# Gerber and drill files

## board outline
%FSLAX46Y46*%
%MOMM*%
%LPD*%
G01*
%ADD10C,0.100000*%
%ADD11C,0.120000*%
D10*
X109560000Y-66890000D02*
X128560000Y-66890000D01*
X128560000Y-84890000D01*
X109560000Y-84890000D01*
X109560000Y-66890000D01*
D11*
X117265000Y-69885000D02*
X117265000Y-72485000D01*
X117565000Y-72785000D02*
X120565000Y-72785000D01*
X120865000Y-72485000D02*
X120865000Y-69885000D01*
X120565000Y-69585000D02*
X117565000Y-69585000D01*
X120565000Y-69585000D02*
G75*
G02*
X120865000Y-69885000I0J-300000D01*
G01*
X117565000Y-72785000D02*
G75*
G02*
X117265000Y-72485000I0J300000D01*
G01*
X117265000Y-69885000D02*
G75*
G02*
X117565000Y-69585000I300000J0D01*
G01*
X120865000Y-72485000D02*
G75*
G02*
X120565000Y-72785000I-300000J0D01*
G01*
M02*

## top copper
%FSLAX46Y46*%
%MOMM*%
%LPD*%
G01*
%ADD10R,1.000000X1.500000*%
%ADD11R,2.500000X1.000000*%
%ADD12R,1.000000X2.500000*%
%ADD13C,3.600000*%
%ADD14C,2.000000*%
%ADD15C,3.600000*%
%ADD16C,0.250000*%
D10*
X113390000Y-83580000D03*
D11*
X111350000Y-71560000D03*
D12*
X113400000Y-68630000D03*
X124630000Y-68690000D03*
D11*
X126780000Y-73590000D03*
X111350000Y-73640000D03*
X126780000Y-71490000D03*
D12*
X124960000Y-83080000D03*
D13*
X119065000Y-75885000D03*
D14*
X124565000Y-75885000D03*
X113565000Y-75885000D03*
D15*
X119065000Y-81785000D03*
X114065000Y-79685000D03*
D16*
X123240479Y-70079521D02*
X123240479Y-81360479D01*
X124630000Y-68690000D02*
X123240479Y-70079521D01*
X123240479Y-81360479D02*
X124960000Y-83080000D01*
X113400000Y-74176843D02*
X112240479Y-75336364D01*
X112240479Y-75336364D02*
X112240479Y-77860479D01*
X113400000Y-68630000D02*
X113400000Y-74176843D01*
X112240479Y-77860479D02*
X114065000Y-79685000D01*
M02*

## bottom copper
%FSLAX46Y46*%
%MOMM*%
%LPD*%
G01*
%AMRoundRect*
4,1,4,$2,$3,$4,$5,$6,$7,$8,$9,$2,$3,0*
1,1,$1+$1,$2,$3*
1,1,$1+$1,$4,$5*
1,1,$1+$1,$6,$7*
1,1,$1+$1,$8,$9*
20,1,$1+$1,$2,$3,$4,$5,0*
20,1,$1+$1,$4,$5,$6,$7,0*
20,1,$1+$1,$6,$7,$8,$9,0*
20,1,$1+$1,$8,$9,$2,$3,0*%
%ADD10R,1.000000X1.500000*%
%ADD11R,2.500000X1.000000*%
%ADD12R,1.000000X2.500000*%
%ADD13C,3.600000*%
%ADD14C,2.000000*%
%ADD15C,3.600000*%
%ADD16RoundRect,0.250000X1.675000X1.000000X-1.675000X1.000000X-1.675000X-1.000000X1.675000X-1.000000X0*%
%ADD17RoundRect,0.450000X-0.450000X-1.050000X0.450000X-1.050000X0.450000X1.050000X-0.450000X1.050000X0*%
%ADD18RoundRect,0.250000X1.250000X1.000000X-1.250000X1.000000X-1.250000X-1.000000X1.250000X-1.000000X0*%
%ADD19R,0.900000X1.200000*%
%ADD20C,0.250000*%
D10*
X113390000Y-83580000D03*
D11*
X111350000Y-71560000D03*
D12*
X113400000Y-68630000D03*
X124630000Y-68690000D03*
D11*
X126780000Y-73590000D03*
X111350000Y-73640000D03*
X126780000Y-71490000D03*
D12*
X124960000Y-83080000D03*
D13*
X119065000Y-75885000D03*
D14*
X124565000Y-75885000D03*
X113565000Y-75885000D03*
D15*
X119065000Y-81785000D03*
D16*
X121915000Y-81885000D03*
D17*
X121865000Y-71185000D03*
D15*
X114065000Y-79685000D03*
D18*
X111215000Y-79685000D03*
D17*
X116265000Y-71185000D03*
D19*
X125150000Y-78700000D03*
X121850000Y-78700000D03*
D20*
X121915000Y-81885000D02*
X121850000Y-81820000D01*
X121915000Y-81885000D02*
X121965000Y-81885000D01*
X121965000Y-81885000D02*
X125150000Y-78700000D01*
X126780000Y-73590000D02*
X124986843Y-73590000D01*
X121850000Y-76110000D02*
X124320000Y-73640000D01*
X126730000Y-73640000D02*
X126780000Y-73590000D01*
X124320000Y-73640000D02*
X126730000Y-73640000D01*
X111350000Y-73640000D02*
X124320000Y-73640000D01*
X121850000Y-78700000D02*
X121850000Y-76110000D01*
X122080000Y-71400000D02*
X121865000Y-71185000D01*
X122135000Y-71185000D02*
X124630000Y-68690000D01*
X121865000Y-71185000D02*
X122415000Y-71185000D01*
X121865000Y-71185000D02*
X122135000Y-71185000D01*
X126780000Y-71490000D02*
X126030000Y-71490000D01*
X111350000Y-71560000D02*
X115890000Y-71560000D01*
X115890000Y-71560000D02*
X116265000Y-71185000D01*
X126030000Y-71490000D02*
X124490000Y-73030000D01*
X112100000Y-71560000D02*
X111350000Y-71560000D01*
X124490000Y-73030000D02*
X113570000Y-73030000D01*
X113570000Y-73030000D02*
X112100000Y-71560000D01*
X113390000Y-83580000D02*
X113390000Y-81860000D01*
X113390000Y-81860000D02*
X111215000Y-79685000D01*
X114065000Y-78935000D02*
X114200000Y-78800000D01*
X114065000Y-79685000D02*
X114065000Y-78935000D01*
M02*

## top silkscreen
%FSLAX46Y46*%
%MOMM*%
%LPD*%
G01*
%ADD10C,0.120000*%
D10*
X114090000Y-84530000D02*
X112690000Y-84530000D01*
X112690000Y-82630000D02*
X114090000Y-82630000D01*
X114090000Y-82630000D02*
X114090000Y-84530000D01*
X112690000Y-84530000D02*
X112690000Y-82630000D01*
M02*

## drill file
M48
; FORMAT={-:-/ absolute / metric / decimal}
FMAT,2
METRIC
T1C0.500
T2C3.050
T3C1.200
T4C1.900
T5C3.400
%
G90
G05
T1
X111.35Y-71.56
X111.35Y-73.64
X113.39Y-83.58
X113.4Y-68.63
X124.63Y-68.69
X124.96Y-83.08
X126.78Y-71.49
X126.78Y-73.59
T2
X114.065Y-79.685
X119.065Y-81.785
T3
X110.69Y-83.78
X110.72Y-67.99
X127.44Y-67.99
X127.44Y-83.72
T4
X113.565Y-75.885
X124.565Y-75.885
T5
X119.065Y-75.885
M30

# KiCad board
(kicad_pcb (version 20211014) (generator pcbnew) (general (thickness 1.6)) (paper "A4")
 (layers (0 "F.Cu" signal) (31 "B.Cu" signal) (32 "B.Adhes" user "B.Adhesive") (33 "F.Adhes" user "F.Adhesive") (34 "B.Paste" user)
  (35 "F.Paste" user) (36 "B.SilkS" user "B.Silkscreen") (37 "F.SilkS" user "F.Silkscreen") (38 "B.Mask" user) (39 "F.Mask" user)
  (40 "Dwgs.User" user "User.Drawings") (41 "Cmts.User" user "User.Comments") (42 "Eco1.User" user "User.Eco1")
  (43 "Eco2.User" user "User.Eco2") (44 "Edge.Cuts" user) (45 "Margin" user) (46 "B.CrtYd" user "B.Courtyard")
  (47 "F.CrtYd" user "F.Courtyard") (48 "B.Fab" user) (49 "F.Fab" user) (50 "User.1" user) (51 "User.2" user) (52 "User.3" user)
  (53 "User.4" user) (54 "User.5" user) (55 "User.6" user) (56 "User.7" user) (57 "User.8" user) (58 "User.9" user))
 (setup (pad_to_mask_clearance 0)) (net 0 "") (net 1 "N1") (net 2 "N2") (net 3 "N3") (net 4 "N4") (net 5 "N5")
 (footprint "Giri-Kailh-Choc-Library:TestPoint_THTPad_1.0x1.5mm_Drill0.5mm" (layer "F.Cu") (at 113.39 83.58 -90)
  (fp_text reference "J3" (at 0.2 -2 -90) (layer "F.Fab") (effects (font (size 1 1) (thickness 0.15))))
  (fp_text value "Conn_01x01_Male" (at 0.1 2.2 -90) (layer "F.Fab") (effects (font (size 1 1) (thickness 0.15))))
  (fp_line (start 0.95 -0.7) (end 0.95 0.7) (layer "F.SilkS") (width 0.12))
  (fp_line (start -0.95 0.7) (end -0.95 -0.7) (layer "F.SilkS") (width 0.12))
  (fp_line (start -0.95 -0.7) (end 0.95 -0.7) (layer "F.SilkS") (width 0.12))
  (fp_line (start 0.95 0.7) (end -0.95 0.7) (layer "F.SilkS") (width 0.12))
  (pad "1" thru_hole rect (at 0 0 270) (size 1.5 1) (drill 0.5) (layers *.Cu *.Mask) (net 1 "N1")))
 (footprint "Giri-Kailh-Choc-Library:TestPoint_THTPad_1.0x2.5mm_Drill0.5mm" (layer "F.Cu") (at 111.35 71.56)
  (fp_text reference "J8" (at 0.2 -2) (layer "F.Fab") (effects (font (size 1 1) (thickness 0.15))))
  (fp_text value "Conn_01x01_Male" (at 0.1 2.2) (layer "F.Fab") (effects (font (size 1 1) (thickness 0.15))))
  (pad "1" thru_hole rect (at 0 0) (size 2.5 1) (drill 0.5) (layers *.Cu *.Mask) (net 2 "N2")))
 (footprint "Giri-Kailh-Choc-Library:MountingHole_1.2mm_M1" (layer "F.Cu") (at 110.69 83.78)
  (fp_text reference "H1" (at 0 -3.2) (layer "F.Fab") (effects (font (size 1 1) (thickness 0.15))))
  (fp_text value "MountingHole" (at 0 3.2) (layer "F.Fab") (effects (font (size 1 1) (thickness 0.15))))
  (pad "" np_thru_hole circle (at 0 0) (size 1.2 1.2) (drill 1.2) (layers F&B.Cu *.Mask)))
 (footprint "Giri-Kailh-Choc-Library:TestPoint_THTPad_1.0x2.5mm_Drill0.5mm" (layer "F.Cu") (at 113.4 68.63 90)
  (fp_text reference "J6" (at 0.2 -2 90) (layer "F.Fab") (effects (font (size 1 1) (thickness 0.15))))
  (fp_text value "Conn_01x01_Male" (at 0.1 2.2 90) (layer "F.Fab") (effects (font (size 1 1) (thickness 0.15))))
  (pad "1" thru_hole rect (at 0 0 90) (size 2.5 1) (drill 0.5) (layers *.Cu *.Mask) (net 1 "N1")))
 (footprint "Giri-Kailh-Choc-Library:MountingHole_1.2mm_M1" (layer "F.Cu") (at 127.44 83.72)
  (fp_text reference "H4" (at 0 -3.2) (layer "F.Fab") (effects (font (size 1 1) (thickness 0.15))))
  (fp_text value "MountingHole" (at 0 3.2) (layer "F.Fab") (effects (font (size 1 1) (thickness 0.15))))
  (pad "" np_thru_hole circle (at 0 0) (size 1.2 1.2) (drill 1.2) (layers F&B.Cu *.Mask)))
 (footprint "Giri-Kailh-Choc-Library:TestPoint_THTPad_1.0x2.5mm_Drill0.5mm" (layer "F.Cu") (at 124.63 68.69 90)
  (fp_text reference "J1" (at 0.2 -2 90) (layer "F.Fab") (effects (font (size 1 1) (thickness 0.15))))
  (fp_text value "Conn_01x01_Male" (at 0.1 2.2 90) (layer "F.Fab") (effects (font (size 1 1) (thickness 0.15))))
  (pad "1" thru_hole rect (at 0 0 90) (size 2.5 1) (drill 0.5) (layers *.Cu *.Mask) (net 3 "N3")))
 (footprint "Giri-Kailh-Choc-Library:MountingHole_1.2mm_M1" (layer "F.Cu") (at 127.44 67.99)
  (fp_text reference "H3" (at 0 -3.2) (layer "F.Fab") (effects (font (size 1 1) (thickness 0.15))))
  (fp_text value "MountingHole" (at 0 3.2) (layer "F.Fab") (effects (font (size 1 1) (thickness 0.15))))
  (pad "" np_thru_hole circle (at 0 0) (size 1.2 1.2) (drill 1.2) (layers F&B.Cu *.Mask)))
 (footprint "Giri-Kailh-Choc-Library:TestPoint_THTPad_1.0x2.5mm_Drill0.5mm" (layer "F.Cu") (at 126.78 73.59)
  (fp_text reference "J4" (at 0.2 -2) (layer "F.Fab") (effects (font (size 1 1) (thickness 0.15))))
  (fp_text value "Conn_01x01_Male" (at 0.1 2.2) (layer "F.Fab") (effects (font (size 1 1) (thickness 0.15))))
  (pad "1" thru_hole rect (at 0 0) (size 2.5 1) (drill 0.5) (layers *.Cu *.Mask) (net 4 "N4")))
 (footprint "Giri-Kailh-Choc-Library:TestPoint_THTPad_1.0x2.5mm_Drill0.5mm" (layer "F.Cu") (at 111.35 73.64)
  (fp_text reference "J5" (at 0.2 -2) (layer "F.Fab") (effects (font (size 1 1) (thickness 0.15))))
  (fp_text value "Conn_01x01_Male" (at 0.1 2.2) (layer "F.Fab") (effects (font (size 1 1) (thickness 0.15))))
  (pad "1" thru_hole rect (at 0 0) (size 2.5 1) (drill 0.5) (layers *.Cu *.Mask) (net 4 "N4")))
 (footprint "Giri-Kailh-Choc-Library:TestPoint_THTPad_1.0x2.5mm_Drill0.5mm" (layer "F.Cu") (at 126.78 71.49)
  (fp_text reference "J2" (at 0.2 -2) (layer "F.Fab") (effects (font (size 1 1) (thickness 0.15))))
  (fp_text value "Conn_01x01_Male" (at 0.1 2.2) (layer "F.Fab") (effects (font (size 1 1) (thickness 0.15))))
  (pad "1" thru_hole rect (at 0 0) (size 2.5 1) (drill 0.5) (layers *.Cu *.Mask) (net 2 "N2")))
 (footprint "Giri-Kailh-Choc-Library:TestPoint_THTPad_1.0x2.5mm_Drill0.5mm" (layer "F.Cu") (at 124.96 83.08 90)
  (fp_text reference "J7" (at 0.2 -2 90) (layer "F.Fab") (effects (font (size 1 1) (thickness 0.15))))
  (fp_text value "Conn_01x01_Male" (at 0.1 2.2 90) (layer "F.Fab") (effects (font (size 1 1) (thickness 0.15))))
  (pad "1" thru_hole rect (at 0 0 90) (size 2.5 1) (drill 0.5) (layers *.Cu *.Mask) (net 3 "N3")))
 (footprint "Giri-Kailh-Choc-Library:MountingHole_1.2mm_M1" (layer "F.Cu") (at 110.72 67.99)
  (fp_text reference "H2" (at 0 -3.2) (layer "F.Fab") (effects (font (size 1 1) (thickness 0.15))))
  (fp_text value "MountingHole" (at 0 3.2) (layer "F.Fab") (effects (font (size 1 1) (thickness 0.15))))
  (pad "" np_thru_hole circle (at 0 0) (size 1.2 1.2) (drill 1.2) (layers F&B.Cu *.Mask)))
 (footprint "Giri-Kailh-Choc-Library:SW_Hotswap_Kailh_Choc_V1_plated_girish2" (layer "F.Cu") (at 119.065 75.885)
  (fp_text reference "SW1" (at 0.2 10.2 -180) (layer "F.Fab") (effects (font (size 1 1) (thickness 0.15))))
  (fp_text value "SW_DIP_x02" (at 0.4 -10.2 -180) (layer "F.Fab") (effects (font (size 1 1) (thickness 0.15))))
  (fp_line (start -1.8 -6) (end -1.8 -3.4) (layer "Edge.Cuts") (width 0.12))
  (fp_line (start -1.5 -3.1) (end 1.5 -3.1) (layer "Edge.Cuts") (width 0.12))
  (fp_line (start 1.8 -3.4) (end 1.8 -6) (layer "Edge.Cuts") (width 0.12))
  (fp_line (start 1.5 -6.3) (end -1.5 -6.3) (layer "Edge.Cuts") (width 0.12))
  (fp_arc (start 1.5 -6.3) (mid 1.712132 -6.212132) (end 1.8 -6) (layer "Edge.Cuts") (width 0.12))
  (fp_arc (start -1.5 -3.1) (mid -1.712132 -3.187868) (end -1.8 -3.4) (layer "Edge.Cuts") (width 0.12))
  (fp_arc (start -1.8 -6) (mid -1.712132 -6.212132) (end -1.5 -6.3) (layer "Edge.Cuts") (width 0.12))
  (fp_arc (start 1.8 -3.4) (mid 1.712132 -3.187868) (end 1.5 -3.1) (layer "Edge.Cuts") (width 0.12))
  (pad "" np_thru_hole circle (at 0 0 180) (size 3.6 3.6) (drill 3.4) (layers F&B.Cu *.Mask))
  (pad "" smd roundrect (at 3.5 6 180) (size 2.55 2.5) (layers "B.Paste" "B.Mask") (roundrect_rratio 0.1))
  (pad "" np_thru_hole circle (at 5.5 0 180) (size 2 2) (drill 1.9) (layers F&B.Cu *.Mask))
  (pad "" np_thru_hole circle (at -5.5 0 180) (size 2 2) (drill 1.9) (layers F&B.Cu *.Mask))
  (pad "" smd roundrect (at -8.5 3.8 180) (size 1.9 2.5) (layers "B.Paste" "B.Mask") (roundrect_rratio 0.1))
  (pad "1" thru_hole circle (at 0 5.9 180) (size 3.6 3.6) (drill 3.05) (layers *.Cu "B.Mask") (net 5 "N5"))
  (pad "1" smd roundrect (at 2.85 6 180) (size 3.85 2.5) (layers "B.Cu" "B.Paste" "B.Mask") (roundrect_rratio 0.1) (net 5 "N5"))
  (pad "2" smd roundrect (at 2.8 -4.7) (size 1.8 3) (layers "B.Cu" "B.Paste" "B.Mask") (roundrect_rratio 0.25) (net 3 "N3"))
  (pad "3" thru_hole circle (at -5 3.8 180) (size 3.6 3.6) (drill 3.05) (layers *.Cu "B.Mask") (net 1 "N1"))
  (pad "3" smd roundrect (at -7.85 3.8 180) (size 3 2.5) (layers "B.Cu" "B.Paste" "B.Mask") (roundrect_rratio 0.1) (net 1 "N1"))
  (pad "4" smd roundrect (at -2.8 -4.7) (size 1.8 3) (layers "B.Cu" "B.Paste" "B.Mask") (roundrect_rratio 0.25) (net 2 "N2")))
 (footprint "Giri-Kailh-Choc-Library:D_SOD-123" (layer "B.Cu") (at 123.5 78.7 180)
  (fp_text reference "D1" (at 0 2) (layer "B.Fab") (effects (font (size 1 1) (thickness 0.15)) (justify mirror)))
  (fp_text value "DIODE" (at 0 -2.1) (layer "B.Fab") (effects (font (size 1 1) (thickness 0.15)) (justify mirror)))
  (pad "1" smd rect (at -1.65 0 180) (size 0.9 1.2) (layers "B.Cu" "B.Paste" "B.Mask") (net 5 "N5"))
  (pad "2" smd rect (at 1.65 0 180) (size 0.9 1.2) (layers "B.Cu" "B.Paste" "B.Mask") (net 4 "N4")))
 (gr_rect (start 109.56 84.89) (end 128.56 66.89) (layer "Edge.Cuts") (width 0.1) (fill none))
 (segment (start 121.915 81.885) (end 121.85 81.82) (width 0.25) (layer "B.Cu") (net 5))
 (segment (start 121.915 81.885) (end 121.965 81.885) (width 0.25) (layer "B.Cu") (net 5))
 (segment (start 121.965 81.885) (end 125.15 78.7) (width 0.25) (layer "B.Cu") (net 5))
 (segment (start 126.78 73.59) (end 124.986843 73.59) (width 0.25) (layer "B.Cu") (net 4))
 (segment (start 121.85 76.11) (end 124.32 73.64) (width 0.25) (layer "B.Cu") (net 4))
 (segment (start 126.73 73.64) (end 126.78 73.59) (width 0.25) (layer "B.Cu") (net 4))
 (segment (start 124.32 73.64) (end 126.73 73.64) (width 0.25) (layer "B.Cu") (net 4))
 (segment (start 111.35 73.64) (end 124.32 73.64) (width 0.25) (layer "B.Cu") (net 4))
 (segment (start 121.85 78.7) (end 121.85 76.11) (width 0.25) (layer "B.Cu") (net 4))
 (segment (start 123.240479 70.079521) (end 123.240479 81.360479) (width 0.25) (layer "F.Cu") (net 3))
 (segment (start 124.63 68.69) (end 123.240479 70.079521) (width 0.25) (layer "F.Cu") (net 3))
 (segment (start 123.240479 81.360479) (end 124.96 83.08) (width 0.25) (layer "F.Cu") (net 3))
 (segment (start 122.08 71.4) (end 121.865 71.185) (width 0.25) (layer "B.Cu") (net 3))
 (segment (start 122.135 71.185) (end 124.63 68.69) (width 0.25) (layer "B.Cu") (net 3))
 (segment (start 121.865 71.185) (end 122.415 71.185) (width 0.25) (layer "B.Cu") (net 3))
 (segment (start 121.865 71.185) (end 122.135 71.185) (width 0.25) (layer "B.Cu") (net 3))
 (segment (start 126.78 71.49) (end 126.03 71.49) (width 0.25) (layer "B.Cu") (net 2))
 (segment (start 111.35 71.56) (end 115.89 71.56) (width 0.25) (layer "B.Cu") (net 2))
 (segment (start 115.89 71.56) (end 116.265 71.185) (width 0.25) (layer "B.Cu") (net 2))
 (segment (start 126.03 71.49) (end 124.49 73.03) (width 0.25) (layer "B.Cu") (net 2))
 (segment (start 112.1 71.56) (end 111.35 71.56) (width 0.25) (layer "B.Cu") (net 2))
 (segment (start 124.49 73.03) (end 113.57 73.03) (width 0.25) (layer "B.Cu") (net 2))
 (segment (start 113.57 73.03) (end 112.1 71.56) (width 0.25) (layer "B.Cu") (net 2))
 (segment (start 113.4 74.176843) (end 112.240479 75.336364) (width 0.25) (layer "F.Cu") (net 1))
 (segment (start 112.240479 75.336364) (end 112.240479 77.860479) (width 0.25) (layer "F.Cu") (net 1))
 (segment (start 113.4 68.63) (end 113.4 74.176843) (width 0.25) (layer "F.Cu") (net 1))
 (segment (start 112.240479 77.860479) (end 114.065 79.685) (width 0.25) (layer "F.Cu") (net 1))
 (segment (start 113.39 83.58) (end 113.39 81.86) (width 0.25) (layer "B.Cu") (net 1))
 (segment (start 113.39 81.86) (end 111.215 79.685) (width 0.25) (layer "B.Cu") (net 1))
 (segment (start 114.065 78.935) (end 114.2 78.8) (width 0.25) (layer "B.Cu") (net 1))
 (segment (start 114.065 79.685) (end 114.065 78.935) (width 0.25) (layer "B.Cu") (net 1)))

